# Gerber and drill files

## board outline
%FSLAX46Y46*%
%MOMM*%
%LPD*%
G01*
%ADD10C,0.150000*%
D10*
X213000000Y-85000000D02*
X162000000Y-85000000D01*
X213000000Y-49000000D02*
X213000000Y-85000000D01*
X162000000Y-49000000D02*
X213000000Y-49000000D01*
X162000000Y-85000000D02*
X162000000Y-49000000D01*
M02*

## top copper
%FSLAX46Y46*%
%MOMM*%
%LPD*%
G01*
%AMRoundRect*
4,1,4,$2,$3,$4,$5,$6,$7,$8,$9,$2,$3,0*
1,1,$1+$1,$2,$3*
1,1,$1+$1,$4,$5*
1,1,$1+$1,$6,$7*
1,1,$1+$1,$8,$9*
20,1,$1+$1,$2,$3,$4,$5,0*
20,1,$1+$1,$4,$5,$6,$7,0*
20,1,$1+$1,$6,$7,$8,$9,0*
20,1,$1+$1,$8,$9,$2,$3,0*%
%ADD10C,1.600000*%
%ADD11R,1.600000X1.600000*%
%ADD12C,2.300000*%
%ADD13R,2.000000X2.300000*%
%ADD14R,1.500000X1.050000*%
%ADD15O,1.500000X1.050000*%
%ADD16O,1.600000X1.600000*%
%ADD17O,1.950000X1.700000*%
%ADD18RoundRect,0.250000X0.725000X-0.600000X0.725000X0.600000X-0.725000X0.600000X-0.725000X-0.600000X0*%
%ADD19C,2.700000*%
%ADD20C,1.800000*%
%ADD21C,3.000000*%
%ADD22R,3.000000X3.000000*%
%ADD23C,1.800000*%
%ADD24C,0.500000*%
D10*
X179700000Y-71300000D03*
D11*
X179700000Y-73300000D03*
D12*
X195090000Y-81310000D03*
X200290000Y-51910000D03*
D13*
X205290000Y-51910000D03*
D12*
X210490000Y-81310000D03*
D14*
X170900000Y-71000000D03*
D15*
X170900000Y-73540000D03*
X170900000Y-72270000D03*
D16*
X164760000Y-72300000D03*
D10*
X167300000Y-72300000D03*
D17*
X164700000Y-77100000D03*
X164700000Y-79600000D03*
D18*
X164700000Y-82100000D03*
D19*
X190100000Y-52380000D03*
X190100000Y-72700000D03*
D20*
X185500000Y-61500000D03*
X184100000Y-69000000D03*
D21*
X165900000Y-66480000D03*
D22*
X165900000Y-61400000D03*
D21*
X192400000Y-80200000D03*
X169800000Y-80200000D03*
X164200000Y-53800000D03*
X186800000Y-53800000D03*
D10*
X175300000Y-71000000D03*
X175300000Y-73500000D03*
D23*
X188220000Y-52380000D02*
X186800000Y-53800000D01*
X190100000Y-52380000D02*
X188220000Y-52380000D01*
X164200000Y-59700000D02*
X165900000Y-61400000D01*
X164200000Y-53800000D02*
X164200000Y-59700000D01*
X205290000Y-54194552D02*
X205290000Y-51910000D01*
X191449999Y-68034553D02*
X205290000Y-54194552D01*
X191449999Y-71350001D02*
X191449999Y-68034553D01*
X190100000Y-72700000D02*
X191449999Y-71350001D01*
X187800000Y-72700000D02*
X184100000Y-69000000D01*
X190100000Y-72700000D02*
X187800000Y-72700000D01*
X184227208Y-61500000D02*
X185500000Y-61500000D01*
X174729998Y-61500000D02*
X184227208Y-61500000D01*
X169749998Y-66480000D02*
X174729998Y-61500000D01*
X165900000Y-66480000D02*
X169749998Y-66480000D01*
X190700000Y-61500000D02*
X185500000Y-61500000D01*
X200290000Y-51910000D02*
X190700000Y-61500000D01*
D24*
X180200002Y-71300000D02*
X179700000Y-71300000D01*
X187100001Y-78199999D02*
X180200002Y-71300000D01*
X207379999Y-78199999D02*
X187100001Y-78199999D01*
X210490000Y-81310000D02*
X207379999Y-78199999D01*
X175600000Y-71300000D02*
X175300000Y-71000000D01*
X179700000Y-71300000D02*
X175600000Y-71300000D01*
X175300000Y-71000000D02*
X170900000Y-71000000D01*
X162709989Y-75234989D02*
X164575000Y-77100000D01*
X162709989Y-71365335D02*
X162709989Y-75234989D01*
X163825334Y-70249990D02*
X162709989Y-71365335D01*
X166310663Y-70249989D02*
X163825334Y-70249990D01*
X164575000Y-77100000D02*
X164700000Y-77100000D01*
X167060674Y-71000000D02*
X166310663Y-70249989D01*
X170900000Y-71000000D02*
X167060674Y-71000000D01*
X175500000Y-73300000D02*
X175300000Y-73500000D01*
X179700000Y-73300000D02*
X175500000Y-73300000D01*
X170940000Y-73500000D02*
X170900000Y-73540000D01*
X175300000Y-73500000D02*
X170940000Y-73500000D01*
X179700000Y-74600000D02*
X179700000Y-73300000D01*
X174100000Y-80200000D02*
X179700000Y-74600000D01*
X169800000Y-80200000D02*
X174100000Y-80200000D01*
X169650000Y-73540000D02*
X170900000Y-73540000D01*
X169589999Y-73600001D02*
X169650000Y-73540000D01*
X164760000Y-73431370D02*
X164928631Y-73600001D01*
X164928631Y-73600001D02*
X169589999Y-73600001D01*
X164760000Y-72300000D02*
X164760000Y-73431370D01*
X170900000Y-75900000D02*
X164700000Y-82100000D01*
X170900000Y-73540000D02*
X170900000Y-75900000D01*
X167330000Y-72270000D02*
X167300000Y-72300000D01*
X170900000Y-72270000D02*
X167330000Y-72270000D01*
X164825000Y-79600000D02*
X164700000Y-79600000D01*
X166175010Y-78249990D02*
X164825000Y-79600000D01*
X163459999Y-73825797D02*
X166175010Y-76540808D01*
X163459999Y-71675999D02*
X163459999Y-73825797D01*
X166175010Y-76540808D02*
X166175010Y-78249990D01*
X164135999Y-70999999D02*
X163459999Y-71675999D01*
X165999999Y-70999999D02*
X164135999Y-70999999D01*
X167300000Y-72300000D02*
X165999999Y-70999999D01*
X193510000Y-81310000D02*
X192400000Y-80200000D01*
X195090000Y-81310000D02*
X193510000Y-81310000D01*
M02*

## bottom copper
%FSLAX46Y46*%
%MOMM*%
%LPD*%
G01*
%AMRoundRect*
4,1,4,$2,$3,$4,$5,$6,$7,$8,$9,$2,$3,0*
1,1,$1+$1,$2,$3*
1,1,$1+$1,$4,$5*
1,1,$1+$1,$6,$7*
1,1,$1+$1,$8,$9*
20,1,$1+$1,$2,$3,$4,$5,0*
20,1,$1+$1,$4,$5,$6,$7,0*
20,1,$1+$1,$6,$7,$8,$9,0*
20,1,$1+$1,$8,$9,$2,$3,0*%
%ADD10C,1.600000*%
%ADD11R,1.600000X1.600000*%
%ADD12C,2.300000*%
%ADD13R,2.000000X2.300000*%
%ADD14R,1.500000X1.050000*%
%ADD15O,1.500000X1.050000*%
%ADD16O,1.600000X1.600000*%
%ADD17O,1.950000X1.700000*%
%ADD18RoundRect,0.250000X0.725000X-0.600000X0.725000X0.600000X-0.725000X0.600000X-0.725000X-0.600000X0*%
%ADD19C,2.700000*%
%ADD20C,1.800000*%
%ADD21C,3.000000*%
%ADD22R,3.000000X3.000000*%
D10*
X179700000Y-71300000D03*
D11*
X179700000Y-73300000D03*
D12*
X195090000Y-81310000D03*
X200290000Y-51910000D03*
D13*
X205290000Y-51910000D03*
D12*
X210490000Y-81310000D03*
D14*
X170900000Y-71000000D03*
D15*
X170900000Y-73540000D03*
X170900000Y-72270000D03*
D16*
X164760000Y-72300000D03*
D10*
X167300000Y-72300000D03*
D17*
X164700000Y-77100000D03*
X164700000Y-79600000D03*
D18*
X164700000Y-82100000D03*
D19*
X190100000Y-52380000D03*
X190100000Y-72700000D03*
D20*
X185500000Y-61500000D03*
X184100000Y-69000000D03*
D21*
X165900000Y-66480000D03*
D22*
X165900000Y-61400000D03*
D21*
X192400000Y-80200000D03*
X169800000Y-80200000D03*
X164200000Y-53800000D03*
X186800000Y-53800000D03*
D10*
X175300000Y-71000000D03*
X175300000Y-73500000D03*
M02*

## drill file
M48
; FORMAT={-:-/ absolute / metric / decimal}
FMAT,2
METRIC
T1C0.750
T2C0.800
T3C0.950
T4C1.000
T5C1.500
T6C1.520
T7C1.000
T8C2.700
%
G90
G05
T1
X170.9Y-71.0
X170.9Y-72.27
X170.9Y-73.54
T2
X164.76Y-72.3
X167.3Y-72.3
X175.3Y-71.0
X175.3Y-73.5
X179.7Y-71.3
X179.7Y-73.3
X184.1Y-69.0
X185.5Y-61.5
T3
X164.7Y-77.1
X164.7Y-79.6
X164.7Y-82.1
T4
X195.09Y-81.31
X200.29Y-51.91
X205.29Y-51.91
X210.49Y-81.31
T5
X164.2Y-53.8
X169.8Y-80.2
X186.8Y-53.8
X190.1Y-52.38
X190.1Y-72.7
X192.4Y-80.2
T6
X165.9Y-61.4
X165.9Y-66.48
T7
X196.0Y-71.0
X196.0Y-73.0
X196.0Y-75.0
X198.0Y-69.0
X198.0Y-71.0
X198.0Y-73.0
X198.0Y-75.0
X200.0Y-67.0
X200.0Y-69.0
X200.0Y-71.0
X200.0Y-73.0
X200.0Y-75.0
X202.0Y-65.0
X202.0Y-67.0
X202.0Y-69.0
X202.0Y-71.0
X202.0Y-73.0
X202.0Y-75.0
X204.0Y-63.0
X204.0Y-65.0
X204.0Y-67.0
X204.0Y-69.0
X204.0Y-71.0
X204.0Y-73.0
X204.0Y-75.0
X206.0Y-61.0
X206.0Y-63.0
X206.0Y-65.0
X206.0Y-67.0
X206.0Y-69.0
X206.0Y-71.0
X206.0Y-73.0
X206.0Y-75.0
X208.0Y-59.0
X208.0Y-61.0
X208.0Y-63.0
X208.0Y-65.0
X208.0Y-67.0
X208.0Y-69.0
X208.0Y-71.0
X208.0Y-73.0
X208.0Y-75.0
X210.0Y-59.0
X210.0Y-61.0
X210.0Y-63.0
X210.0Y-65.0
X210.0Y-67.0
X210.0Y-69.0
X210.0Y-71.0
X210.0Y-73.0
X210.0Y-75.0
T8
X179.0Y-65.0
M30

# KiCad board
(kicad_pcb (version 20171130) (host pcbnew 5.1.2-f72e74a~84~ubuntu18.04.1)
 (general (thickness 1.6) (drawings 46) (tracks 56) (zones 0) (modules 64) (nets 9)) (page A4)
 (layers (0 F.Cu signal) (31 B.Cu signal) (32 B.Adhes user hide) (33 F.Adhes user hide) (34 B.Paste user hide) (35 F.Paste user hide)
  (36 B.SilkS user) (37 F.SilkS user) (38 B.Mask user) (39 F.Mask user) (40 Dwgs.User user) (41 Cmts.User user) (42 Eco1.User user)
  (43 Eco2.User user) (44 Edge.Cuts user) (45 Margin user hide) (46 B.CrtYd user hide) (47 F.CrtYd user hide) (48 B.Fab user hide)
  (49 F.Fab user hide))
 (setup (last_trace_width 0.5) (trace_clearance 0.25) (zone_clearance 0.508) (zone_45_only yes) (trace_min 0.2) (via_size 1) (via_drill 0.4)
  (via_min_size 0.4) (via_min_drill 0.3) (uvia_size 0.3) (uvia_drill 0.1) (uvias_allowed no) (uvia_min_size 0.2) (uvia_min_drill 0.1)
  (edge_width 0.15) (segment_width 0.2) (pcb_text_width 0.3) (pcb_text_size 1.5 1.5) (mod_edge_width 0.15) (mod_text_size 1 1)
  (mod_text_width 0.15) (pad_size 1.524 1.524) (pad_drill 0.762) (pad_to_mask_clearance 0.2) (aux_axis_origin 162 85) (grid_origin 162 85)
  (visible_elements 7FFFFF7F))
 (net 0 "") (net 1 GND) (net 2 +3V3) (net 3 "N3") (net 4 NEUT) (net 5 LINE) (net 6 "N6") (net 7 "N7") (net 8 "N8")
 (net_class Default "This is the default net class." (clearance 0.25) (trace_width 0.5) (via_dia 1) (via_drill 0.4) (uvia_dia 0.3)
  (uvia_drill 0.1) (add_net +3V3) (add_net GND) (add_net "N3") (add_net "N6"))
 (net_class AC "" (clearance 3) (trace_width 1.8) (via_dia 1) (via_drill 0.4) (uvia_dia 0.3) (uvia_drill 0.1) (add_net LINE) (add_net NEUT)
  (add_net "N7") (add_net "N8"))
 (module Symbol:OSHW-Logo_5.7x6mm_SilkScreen (layer B.Cu) (at 203.1 79.7 180)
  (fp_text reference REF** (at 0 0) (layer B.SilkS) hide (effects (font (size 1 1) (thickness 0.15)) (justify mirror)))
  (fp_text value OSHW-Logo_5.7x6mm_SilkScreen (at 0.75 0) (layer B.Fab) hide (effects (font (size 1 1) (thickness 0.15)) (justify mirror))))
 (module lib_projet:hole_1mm (layer F.Cu) (at 210 75)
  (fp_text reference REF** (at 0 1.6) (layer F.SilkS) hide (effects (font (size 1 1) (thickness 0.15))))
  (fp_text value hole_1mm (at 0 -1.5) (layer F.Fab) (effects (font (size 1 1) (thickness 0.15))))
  (pad "" np_thru_hole circle (at 0 0) (size 1 1) (drill 1) (layers *.Cu *.Mask)))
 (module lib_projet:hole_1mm (layer F.Cu) (at 208 75)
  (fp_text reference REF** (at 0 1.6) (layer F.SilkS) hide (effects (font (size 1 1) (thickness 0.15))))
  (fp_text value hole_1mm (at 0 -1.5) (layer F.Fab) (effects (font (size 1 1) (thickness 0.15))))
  (pad "" np_thru_hole circle (at 0 0) (size 1 1) (drill 1) (layers *.Cu *.Mask)))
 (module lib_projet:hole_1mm (layer F.Cu) (at 206 75)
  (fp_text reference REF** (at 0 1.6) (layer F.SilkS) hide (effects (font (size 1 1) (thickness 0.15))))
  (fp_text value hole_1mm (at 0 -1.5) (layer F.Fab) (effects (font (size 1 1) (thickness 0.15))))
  (pad "" np_thru_hole circle (at 0 0) (size 1 1) (drill 1) (layers *.Cu *.Mask)))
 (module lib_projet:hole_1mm (layer F.Cu) (at 204 75)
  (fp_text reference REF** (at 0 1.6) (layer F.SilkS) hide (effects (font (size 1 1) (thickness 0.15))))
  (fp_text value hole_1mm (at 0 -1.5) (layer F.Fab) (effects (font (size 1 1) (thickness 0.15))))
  (pad "" np_thru_hole circle (at 0 0) (size 1 1) (drill 1) (layers *.Cu *.Mask)))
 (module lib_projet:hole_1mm (layer F.Cu) (at 202 75)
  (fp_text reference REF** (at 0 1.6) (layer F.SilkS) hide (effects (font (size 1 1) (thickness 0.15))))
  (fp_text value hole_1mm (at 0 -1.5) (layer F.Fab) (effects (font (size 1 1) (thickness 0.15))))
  (pad "" np_thru_hole circle (at 0 0) (size 1 1) (drill 1) (layers *.Cu *.Mask)))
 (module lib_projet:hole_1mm (layer F.Cu) (at 200 75)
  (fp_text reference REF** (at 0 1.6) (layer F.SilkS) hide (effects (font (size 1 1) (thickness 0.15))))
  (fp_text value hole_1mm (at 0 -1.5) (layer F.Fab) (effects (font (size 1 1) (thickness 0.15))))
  (pad "" np_thru_hole circle (at 0 0) (size 1 1) (drill 1) (layers *.Cu *.Mask)))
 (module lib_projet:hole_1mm (layer F.Cu) (at 198 75)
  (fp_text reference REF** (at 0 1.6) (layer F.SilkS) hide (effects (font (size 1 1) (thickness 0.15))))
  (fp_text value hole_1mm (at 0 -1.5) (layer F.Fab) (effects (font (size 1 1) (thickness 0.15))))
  (pad "" np_thru_hole circle (at 0 0) (size 1 1) (drill 1) (layers *.Cu *.Mask)))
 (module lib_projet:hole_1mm (layer F.Cu) (at 196 75)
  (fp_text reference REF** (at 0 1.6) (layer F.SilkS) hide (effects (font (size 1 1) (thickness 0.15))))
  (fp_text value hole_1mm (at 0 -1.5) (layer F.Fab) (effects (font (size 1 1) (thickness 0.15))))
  (pad "" np_thru_hole circle (at 0 0) (size 1 1) (drill 1) (layers *.Cu *.Mask)))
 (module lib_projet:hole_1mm (layer F.Cu) (at 210 73)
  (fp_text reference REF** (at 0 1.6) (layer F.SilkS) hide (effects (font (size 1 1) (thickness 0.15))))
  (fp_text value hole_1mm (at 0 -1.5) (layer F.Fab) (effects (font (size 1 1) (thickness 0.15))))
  (pad "" np_thru_hole circle (at 0 0) (size 1 1) (drill 1) (layers *.Cu *.Mask)))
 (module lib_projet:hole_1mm (layer F.Cu) (at 208 73)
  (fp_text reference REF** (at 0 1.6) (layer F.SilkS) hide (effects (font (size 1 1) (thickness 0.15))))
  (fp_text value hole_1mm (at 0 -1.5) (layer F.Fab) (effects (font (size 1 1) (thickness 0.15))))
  (pad "" np_thru_hole circle (at 0 0) (size 1 1) (drill 1) (layers *.Cu *.Mask)))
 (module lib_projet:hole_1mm (layer F.Cu) (at 206 73)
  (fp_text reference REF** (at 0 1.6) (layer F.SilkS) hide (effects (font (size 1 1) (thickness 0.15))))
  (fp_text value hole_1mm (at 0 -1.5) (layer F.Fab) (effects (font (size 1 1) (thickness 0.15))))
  (pad "" np_thru_hole circle (at 0 0) (size 1 1) (drill 1) (layers *.Cu *.Mask)))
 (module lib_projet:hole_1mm (layer F.Cu) (at 204 73)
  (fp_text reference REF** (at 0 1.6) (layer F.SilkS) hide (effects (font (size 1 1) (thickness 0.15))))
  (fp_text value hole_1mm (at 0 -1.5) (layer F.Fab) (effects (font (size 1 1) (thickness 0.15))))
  (pad "" np_thru_hole circle (at 0 0) (size 1 1) (drill 1) (layers *.Cu *.Mask)))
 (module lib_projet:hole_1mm (layer F.Cu) (at 202 73)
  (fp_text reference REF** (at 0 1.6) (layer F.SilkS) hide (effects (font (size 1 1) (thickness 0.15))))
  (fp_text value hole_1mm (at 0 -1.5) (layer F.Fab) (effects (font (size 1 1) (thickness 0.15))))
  (pad "" np_thru_hole circle (at 0 0) (size 1 1) (drill 1) (layers *.Cu *.Mask)))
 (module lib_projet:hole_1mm (layer F.Cu) (at 200 73)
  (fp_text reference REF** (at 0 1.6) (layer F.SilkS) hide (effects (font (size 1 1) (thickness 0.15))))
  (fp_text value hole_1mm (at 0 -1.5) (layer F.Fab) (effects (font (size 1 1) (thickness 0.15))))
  (pad "" np_thru_hole circle (at 0 0) (size 1 1) (drill 1) (layers *.Cu *.Mask)))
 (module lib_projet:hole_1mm (layer F.Cu) (at 198 73)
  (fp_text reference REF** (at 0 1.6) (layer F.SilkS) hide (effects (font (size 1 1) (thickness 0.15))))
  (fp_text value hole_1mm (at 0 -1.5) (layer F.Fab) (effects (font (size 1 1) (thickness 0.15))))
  (pad "" np_thru_hole circle (at 0 0) (size 1 1) (drill 1) (layers *.Cu *.Mask)))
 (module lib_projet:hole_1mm (layer F.Cu) (at 196 73)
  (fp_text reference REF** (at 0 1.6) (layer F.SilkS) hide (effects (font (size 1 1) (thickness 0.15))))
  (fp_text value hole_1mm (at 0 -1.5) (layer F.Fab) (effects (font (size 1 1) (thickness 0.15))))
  (pad "" np_thru_hole circle (at 0 0) (size 1 1) (drill 1) (layers *.Cu *.Mask)))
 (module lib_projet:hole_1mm (layer F.Cu) (at 210 71)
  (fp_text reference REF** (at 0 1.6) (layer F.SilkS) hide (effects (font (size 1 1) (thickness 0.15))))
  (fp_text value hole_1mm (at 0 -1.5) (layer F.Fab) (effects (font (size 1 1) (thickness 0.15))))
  (pad "" np_thru_hole circle (at 0 0) (size 1 1) (drill 1) (layers *.Cu *.Mask)))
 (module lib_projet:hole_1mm (layer F.Cu) (at 208 71)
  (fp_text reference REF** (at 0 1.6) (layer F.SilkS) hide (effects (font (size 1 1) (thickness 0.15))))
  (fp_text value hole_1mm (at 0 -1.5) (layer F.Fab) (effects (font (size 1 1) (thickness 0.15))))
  (pad "" np_thru_hole circle (at 0 0) (size 1 1) (drill 1) (layers *.Cu *.Mask)))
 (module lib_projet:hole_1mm (layer F.Cu) (at 206 71)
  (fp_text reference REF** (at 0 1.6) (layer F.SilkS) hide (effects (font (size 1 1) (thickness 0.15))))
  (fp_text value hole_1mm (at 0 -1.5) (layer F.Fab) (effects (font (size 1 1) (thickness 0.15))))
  (pad "" np_thru_hole circle (at 0 0) (size 1 1) (drill 1) (layers *.Cu *.Mask)))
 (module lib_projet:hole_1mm (layer F.Cu) (at 204 71)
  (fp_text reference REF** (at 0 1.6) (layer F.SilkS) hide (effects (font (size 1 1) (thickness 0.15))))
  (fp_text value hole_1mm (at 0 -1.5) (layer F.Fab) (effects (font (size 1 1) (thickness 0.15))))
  (pad "" np_thru_hole circle (at 0 0) (size 1 1) (drill 1) (layers *.Cu *.Mask)))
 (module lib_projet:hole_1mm (layer F.Cu) (at 202 71)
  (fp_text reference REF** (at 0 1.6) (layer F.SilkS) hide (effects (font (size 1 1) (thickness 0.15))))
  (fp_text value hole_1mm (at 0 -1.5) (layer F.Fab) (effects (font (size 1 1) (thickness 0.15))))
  (pad "" np_thru_hole circle (at 0 0) (size 1 1) (drill 1) (layers *.Cu *.Mask)))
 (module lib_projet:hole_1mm (layer F.Cu) (at 200 71)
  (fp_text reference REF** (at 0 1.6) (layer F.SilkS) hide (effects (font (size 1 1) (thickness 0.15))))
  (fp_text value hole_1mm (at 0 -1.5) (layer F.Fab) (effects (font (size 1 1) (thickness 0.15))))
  (pad "" np_thru_hole circle (at 0 0) (size 1 1) (drill 1) (layers *.Cu *.Mask)))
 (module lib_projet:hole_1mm (layer F.Cu) (at 198 71)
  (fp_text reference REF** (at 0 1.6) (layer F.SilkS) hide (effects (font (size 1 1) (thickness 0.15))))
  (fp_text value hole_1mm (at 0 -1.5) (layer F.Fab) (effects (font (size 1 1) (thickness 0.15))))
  (pad "" np_thru_hole circle (at 0 0) (size 1 1) (drill 1) (layers *.Cu *.Mask)))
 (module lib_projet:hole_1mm (layer F.Cu) (at 196 71)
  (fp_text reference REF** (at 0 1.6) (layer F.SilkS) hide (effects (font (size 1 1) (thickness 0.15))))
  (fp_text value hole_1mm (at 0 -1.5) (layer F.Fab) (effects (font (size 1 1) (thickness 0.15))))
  (pad "" np_thru_hole circle (at 0 0) (size 1 1) (drill 1) (layers *.Cu *.Mask)))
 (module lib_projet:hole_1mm (layer F.Cu) (at 210 69)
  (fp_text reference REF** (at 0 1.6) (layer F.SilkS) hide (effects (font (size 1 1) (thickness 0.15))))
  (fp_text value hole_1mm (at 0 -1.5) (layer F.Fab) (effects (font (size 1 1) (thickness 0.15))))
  (pad "" np_thru_hole circle (at 0 0) (size 1 1) (drill 1) (layers *.Cu *.Mask)))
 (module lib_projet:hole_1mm (layer F.Cu) (at 208 69)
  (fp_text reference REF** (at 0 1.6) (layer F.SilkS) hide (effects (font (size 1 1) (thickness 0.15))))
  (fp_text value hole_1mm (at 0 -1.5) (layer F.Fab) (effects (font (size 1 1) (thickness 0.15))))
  (pad "" np_thru_hole circle (at 0 0) (size 1 1) (drill 1) (layers *.Cu *.Mask)))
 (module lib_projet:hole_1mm (layer F.Cu) (at 206 69)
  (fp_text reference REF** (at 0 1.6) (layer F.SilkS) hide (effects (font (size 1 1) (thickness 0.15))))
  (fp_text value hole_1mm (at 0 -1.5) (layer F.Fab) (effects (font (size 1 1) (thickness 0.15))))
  (pad "" np_thru_hole circle (at 0 0) (size 1 1) (drill 1) (layers *.Cu *.Mask)))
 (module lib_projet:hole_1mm (layer F.Cu) (at 204 69)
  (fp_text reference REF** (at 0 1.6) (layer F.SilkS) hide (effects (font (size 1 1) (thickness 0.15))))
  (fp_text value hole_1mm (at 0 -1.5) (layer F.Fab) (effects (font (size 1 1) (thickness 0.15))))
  (pad "" np_thru_hole circle (at 0 0) (size 1 1) (drill 1) (layers *.Cu *.Mask)))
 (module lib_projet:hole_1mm (layer F.Cu) (at 202 69)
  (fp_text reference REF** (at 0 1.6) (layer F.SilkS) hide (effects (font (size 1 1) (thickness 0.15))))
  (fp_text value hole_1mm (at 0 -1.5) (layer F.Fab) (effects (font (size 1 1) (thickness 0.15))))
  (pad "" np_thru_hole circle (at 0 0) (size 1 1) (drill 1) (layers *.Cu *.Mask)))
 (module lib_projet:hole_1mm (layer F.Cu) (at 200 69)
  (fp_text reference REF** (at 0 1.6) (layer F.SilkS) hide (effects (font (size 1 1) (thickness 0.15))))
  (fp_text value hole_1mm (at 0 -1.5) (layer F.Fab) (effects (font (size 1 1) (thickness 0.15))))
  (pad "" np_thru_hole circle (at 0 0) (size 1 1) (drill 1) (layers *.Cu *.Mask)))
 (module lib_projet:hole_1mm (layer F.Cu) (at 198 69)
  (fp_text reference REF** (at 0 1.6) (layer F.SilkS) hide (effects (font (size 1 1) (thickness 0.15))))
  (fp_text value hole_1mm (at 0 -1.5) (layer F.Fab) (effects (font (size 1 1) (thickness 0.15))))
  (pad "" np_thru_hole circle (at 0 0) (size 1 1) (drill 1) (layers *.Cu *.Mask)))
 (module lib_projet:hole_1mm (layer F.Cu) (at 210 67)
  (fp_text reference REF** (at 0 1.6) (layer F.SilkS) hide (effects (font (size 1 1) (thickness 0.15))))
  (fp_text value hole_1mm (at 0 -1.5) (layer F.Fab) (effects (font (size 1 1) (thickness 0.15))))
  (pad "" np_thru_hole circle (at 0 0) (size 1 1) (drill 1) (layers *.Cu *.Mask)))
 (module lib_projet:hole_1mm (layer F.Cu) (at 208 67)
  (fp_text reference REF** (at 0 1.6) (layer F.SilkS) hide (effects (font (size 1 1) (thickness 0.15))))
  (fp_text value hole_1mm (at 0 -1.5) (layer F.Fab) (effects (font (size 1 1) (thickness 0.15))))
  (pad "" np_thru_hole circle (at 0 0) (size 1 1) (drill 1) (layers *.Cu *.Mask)))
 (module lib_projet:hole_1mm (layer F.Cu) (at 206 67)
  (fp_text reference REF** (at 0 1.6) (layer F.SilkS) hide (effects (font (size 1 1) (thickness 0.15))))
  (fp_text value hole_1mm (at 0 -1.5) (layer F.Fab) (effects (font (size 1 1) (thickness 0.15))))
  (pad "" np_thru_hole circle (at 0 0) (size 1 1) (drill 1) (layers *.Cu *.Mask)))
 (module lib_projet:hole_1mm (layer F.Cu) (at 204 67)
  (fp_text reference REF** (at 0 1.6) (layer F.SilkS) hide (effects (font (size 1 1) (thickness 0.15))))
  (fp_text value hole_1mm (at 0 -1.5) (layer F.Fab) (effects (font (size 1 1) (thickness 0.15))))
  (pad "" np_thru_hole circle (at 0 0) (size 1 1) (drill 1) (layers *.Cu *.Mask)))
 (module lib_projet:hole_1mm (layer F.Cu) (at 202 67)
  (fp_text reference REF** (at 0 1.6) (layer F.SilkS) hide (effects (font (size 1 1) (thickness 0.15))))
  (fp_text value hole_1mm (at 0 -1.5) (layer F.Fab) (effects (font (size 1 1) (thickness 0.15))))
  (pad "" np_thru_hole circle (at 0 0) (size 1 1) (drill 1) (layers *.Cu *.Mask)))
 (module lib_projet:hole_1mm (layer F.Cu) (at 200 67)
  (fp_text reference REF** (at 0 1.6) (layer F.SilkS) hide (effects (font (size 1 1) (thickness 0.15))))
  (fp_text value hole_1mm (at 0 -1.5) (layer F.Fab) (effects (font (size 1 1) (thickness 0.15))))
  (pad "" np_thru_hole circle (at 0 0) (size 1 1) (drill 1) (layers *.Cu *.Mask)))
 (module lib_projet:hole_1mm (layer F.Cu) (at 210 65)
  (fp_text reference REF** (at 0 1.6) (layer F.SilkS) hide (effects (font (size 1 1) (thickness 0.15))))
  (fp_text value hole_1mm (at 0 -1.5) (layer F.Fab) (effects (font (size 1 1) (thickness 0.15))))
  (pad "" np_thru_hole circle (at 0 0) (size 1 1) (drill 1) (layers *.Cu *.Mask)))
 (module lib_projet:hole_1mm (layer F.Cu) (at 208 65)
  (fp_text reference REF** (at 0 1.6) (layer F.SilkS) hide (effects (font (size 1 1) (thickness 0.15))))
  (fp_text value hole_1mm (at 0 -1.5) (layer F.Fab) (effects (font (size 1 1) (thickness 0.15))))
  (pad "" np_thru_hole circle (at 0 0) (size 1 1) (drill 1) (layers *.Cu *.Mask)))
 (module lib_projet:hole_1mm (layer F.Cu) (at 206 65)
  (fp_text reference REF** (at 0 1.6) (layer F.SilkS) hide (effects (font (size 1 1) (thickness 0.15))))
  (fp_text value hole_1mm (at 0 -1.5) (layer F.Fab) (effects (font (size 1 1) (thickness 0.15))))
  (pad "" np_thru_hole circle (at 0 0) (size 1 1) (drill 1) (layers *.Cu *.Mask)))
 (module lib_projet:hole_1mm (layer F.Cu) (at 204 65)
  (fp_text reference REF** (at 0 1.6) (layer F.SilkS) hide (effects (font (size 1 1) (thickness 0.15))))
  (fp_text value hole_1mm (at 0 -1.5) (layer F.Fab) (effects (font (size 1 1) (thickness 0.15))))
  (pad "" np_thru_hole circle (at 0 0) (size 1 1) (drill 1) (layers *.Cu *.Mask)))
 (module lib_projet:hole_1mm (layer F.Cu) (at 202 65)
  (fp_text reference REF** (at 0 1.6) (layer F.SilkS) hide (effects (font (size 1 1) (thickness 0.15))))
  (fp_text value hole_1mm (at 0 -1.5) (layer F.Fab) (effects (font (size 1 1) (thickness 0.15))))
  (pad "" np_thru_hole circle (at 0 0) (size 1 1) (drill 1) (layers *.Cu *.Mask)))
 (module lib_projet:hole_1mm (layer F.Cu) (at 210 63)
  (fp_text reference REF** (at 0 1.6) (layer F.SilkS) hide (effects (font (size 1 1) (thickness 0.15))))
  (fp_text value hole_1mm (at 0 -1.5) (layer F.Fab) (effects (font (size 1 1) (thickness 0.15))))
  (pad "" np_thru_hole circle (at 0 0) (size 1 1) (drill 1) (layers *.Cu *.Mask)))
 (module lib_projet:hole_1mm (layer F.Cu) (at 208 63)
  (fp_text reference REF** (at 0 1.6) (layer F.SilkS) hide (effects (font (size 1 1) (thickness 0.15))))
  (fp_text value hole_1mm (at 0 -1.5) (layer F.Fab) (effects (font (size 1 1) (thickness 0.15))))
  (pad "" np_thru_hole circle (at 0 0) (size 1 1) (drill 1) (layers *.Cu *.Mask)))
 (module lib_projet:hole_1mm (layer F.Cu) (at 206 63)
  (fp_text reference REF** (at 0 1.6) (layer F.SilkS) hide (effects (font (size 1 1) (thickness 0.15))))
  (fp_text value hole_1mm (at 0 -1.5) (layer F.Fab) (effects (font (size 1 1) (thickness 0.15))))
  (pad "" np_thru_hole circle (at 0 0) (size 1 1) (drill 1) (layers *.Cu *.Mask)))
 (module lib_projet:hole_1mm (layer F.Cu) (at 204 63)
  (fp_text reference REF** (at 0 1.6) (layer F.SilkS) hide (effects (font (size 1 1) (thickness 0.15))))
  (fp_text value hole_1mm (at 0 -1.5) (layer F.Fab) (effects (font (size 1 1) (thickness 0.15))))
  (pad "" np_thru_hole circle (at 0 0) (size 1 1) (drill 1) (layers *.Cu *.Mask)))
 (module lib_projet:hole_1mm (layer F.Cu) (at 210 61)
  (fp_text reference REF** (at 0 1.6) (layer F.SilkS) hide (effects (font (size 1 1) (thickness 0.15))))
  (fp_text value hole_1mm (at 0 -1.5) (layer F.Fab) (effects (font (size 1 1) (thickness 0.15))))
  (pad "" np_thru_hole circle (at 0 0) (size 1 1) (drill 1) (layers *.Cu *.Mask)))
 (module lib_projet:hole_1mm (layer F.Cu) (at 208 61)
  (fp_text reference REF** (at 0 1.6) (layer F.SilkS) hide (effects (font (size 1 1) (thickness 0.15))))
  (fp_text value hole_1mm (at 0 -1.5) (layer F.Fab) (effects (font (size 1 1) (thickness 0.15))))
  (pad "" np_thru_hole circle (at 0 0) (size 1 1) (drill 1) (layers *.Cu *.Mask)))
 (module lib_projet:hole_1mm (layer F.Cu) (at 206 61)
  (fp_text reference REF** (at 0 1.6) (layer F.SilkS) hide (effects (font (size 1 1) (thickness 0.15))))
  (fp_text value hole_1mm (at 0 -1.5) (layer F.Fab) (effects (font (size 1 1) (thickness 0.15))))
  (pad "" np_thru_hole circle (at 0 0) (size 1 1) (drill 1) (layers *.Cu *.Mask)))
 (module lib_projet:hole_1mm (layer F.Cu) (at 210 59)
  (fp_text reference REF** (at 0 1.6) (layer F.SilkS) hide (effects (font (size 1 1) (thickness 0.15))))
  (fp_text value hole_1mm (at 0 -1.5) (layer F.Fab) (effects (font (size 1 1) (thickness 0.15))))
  (pad "" np_thru_hole circle (at 0 0) (size 1 1) (drill 1) (layers *.Cu *.Mask)))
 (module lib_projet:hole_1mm (layer F.Cu) (at 208 59)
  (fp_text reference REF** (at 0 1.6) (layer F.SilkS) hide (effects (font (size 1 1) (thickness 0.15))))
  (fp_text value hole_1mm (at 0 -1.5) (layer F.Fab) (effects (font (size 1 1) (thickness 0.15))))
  (pad "" np_thru_hole circle (at 0 0) (size 1 1) (drill 1) (layers *.Cu *.Mask)))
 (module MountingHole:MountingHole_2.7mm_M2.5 (layer F.Cu) (at 179 65)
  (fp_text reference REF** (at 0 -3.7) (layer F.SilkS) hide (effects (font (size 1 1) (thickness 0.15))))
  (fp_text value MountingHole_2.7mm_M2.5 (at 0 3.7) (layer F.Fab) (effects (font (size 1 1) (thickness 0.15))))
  (pad 1 np_thru_hole circle (at 0 0) (size 2.7 2.7) (drill 2.7) (layers *.Cu *.Mask)))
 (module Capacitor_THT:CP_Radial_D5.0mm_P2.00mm (layer F.Cu) (at 179.7 73.3 90)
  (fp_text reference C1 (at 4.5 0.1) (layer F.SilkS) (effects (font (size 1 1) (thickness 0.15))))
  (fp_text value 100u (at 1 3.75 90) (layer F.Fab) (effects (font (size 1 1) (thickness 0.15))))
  (pad 2 thru_hole circle (at 2 0 90) (size 1.6 1.6) (drill 0.8) (layers *.Cu *.Mask) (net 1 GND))
  (pad 1 thru_hole rect (at 0 0 90) (size 1.6 1.6) (drill 0.8) (layers *.Cu *.Mask) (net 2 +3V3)))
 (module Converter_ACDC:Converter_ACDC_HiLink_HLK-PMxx (layer F.Cu) (at 205.29 51.91 270)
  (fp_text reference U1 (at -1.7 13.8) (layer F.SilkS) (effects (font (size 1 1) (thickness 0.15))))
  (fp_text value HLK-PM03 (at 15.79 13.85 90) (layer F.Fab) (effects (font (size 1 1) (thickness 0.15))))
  (pad 4 thru_hole circle (at 29.4 10.2 270) (size 2.3 2.3) (drill 1) (layers *.Cu *.Mask) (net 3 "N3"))
  (pad 2 thru_hole circle (at 0 5 270) (size 2.3 2.3) (drill 1) (layers *.Cu *.Mask) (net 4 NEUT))
  (pad 1 thru_hole rect (at 0 0 270) (size 2.3 2) (drill 1) (layers *.Cu *.Mask) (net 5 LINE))
  (pad 3 thru_hole circle (at 29.4 -5.2 270) (size 2.3 2.3) (drill 1) (layers *.Cu *.Mask) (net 1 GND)))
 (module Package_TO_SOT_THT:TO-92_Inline (layer F.Cu) (at 170.9 71 270)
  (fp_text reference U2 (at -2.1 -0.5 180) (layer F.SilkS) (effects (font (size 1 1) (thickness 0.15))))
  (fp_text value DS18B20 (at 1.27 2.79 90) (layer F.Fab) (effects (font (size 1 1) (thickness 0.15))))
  (pad 1 thru_hole rect (at 0 0 270) (size 1.05 1.5) (drill 0.75) (layers *.Cu *.Mask) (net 1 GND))
  (pad 3 thru_hole oval (at 2.54 0 270) (size 1.05 1.5) (drill 0.75) (layers *.Cu *.Mask) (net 2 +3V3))
  (pad 2 thru_hole oval (at 1.27 0 270) (size 1.05 1.5) (drill 0.75) (layers *.Cu *.Mask) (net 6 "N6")))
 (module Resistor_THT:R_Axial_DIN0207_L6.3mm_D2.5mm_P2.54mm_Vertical (layer F.Cu) (at 167.3 72.3 180)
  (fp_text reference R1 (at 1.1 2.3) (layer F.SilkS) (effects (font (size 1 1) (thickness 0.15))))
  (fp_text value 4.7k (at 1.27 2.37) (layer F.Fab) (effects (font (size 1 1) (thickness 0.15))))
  (pad 2 thru_hole oval (at 2.54 0 180) (size 1.6 1.6) (drill 0.8) (layers *.Cu *.Mask) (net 2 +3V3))
  (pad 1 thru_hole circle (at 0 0 180) (size 1.6 1.6) (drill 0.8) (layers *.Cu *.Mask) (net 6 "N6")))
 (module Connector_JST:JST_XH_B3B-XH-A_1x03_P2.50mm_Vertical (layer F.Cu) (at 164.7 82.1 90)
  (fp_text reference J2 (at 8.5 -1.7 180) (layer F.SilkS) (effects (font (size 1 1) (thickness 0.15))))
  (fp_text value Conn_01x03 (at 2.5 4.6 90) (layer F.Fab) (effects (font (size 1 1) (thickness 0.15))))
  (pad 3 thru_hole oval (at 5 0 90) (size 1.7 1.95) (drill 0.95) (layers *.Cu *.Mask) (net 1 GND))
  (pad 2 thru_hole oval (at 2.5 0 90) (size 1.7 1.95) (drill 0.95) (layers *.Cu *.Mask) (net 6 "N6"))
  (pad 1 thru_hole roundrect (at 0 0 90) (size 1.7 1.95) (drill 0.95) (layers *.Cu *.Mask) (roundrect_rratio 0.147059) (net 2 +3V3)))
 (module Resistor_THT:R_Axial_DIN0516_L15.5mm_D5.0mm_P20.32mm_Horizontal (layer F.Cu) (at 190.1 72.7 90)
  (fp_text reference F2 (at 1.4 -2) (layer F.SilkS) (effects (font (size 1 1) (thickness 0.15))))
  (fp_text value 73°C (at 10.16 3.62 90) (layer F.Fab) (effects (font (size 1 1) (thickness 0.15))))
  (pad 2 thru_hole circle (at 20.32 0 90) (size 2.7 2.7) (drill 1.5) (layers *.Cu *.Mask) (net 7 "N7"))
  (pad 1 thru_hole circle (at 0 0 90) (size 2.7 2.7) (drill 1.5) (layers *.Cu *.Mask) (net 5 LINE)))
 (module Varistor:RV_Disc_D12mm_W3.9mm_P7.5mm (layer F.Cu) (at 184.1 69 90)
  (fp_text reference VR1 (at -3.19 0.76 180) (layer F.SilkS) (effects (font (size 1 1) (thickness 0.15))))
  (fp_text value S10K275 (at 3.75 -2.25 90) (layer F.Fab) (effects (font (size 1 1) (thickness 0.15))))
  (pad 2 thru_hole circle (at 7.5 1.4 90) (size 1.8 1.8) (drill 0.8) (layers *.Cu *.Mask) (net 4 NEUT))
  (pad 1 thru_hole circle (at 0 0 90) (size 1.8 1.8) (drill 0.8) (layers *.Cu *.Mask) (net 5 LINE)))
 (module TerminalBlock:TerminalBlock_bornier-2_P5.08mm (layer F.Cu) (at 165.9 61.4 270)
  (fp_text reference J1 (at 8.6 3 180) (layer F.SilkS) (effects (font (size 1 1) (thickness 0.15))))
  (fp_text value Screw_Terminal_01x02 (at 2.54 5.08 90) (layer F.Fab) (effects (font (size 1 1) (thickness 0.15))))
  (pad 2 thru_hole circle (at 5.08 0 270) (size 3 3) (drill 1.52) (layers *.Cu *.Mask) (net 4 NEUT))
  (pad 1 thru_hole rect (at 0 0 270) (size 3 3) (drill 1.52) (layers *.Cu *.Mask) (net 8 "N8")))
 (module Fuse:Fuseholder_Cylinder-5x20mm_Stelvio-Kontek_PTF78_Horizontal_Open (layer F.Cu) (at 169.8 80.2)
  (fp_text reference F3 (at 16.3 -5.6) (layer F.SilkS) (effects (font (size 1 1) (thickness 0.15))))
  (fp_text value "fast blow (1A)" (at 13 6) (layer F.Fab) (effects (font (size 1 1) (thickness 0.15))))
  (pad 2 thru_hole circle (at 22.6 0) (size 3 3) (drill 1.5) (layers *.Cu *.Mask) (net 3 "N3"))
  (pad 1 thru_hole circle (at 0 0) (size 3 3) (drill 1.5) (layers *.Cu *.Mask) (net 2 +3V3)))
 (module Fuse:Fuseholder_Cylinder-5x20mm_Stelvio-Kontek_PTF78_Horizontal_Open (layer F.Cu) (at 186.8 53.8 180)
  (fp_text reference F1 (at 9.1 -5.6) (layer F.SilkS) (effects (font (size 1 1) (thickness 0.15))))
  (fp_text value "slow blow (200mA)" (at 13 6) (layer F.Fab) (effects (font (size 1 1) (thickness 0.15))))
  (pad 2 thru_hole circle (at 22.6 0 180) (size 3 3) (drill 1.5) (layers *.Cu *.Mask) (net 8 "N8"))
  (pad 1 thru_hole circle (at 0 0 180) (size 3 3) (drill 1.5) (layers *.Cu *.Mask) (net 7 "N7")))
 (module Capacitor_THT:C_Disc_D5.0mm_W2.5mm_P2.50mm (layer F.Cu) (at 175.3 73.5 90)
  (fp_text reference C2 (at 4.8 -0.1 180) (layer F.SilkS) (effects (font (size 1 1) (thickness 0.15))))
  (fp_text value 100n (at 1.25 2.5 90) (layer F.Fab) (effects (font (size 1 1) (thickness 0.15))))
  (pad 2 thru_hole circle (at 2.5 0 90) (size 1.6 1.6) (drill 0.8) (layers *.Cu *.Mask) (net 1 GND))
  (pad 1 thru_hole circle (at 0 0 90) (size 1.6 1.6) (drill 0.8) (layers *.Cu *.Mask) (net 2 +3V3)))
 (gr_line (start 213 85) (end 162 85) (layer Edge.Cuts) (width 0.15))
 (gr_line (start 213 49) (end 213 85) (layer Edge.Cuts) (width 0.15))
 (gr_line (start 162 49) (end 213 49) (layer Edge.Cuts) (width 0.15))
 (gr_line (start 162 85) (end 162 49) (layer Edge.Cuts) (width 0.15))
 (segment (start 188.22 52.38) (end 186.8 53.8) (width 1.8) (layer F.Cu) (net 7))
 (segment (start 190.1 52.38) (end 188.22 52.38) (width 1.8) (layer F.Cu) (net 7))
 (segment (start 164.2 59.7) (end 165.9 61.4) (width 1.8) (layer F.Cu) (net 8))
 (segment (start 164.2 53.8) (end 164.2 59.7) (width 1.8) (layer F.Cu) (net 8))
 (segment (start 205.29 54.194552) (end 205.29 51.91) (width 1.8) (layer F.Cu) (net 5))
 (segment (start 191.449999 68.034553) (end 205.29 54.194552) (width 1.8) (layer F.Cu) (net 5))
 (segment (start 191.449999 71.350001) (end 191.449999 68.034553) (width 1.8) (layer F.Cu) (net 5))
 (segment (start 190.1 72.7) (end 191.449999 71.350001) (width 1.8) (layer F.Cu) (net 5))
 (segment (start 187.8 72.7) (end 184.1 69) (width 1.8) (layer F.Cu) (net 5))
 (segment (start 190.1 72.7) (end 187.8 72.7) (width 1.8) (layer F.Cu) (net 5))
 (segment (start 184.227208 61.5) (end 185.5 61.5) (width 1.8) (layer F.Cu) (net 4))
 (segment (start 174.729998 61.5) (end 184.227208 61.5) (width 1.8) (layer F.Cu) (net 4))
 (segment (start 169.749998 66.48) (end 174.729998 61.5) (width 1.8) (layer F.Cu) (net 4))
 (segment (start 165.9 66.48) (end 169.749998 66.48) (width 1.8) (layer F.Cu) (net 4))
 (segment (start 190.7 61.5) (end 185.5 61.5) (width 1.8) (layer F.Cu) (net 4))
 (segment (start 200.29 51.91) (end 190.7 61.5) (width 1.8) (layer F.Cu) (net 4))
 (segment (start 180.200002 71.3) (end 179.7 71.3) (width 0.5) (layer F.Cu) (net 1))
 (segment (start 187.100001 78.199999) (end 180.200002 71.3) (width 0.5) (layer F.Cu) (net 1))
 (segment (start 207.379999 78.199999) (end 187.100001 78.199999) (width 0.5) (layer F.Cu) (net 1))
 (segment (start 210.49 81.31) (end 207.379999 78.199999) (width 0.5) (layer F.Cu) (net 1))
 (segment (start 175.6 71.3) (end 175.3 71) (width 0.5) (layer F.Cu) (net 1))
 (segment (start 179.7 71.3) (end 175.6 71.3) (width 0.5) (layer F.Cu) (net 1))
 (segment (start 175.3 71) (end 170.9 71) (width 0.5) (layer F.Cu) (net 1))
 (segment (start 162.709989 75.234989) (end 164.575 77.1) (width 0.5) (layer F.Cu) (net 1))
 (segment (start 162.709989 71.365335) (end 162.709989 75.234989) (width 0.5) (layer F.Cu) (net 1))
 (segment (start 163.825334 70.24999) (end 162.709989 71.365335) (width 0.5) (layer F.Cu) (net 1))
 (segment (start 166.310663 70.249989) (end 163.825334 70.24999) (width 0.5) (layer F.Cu) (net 1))
 (segment (start 164.575 77.1) (end 164.7 77.1) (width 0.5) (layer F.Cu) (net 1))
 (segment (start 167.060674 71) (end 166.310663 70.249989) (width 0.5) (layer F.Cu) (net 1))
 (segment (start 170.9 71) (end 167.060674 71) (width 0.5) (layer F.Cu) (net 1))
 (segment (start 175.5 73.3) (end 175.3 73.5) (width 0.5) (layer F.Cu) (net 2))
 (segment (start 179.7 73.3) (end 175.5 73.3) (width 0.5) (layer F.Cu) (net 2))
 (segment (start 170.94 73.5) (end 170.9 73.54) (width 0.5) (layer F.Cu) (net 2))
 (segment (start 175.3 73.5) (end 170.94 73.5) (width 0.5) (layer F.Cu) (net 2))
 (segment (start 179.7 74.6) (end 179.7 73.3) (width 0.5) (layer F.Cu) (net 2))
 (segment (start 174.1 80.2) (end 179.7 74.6) (width 0.5) (layer F.Cu) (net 2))
 (segment (start 169.8 80.2) (end 174.1 80.2) (width 0.5) (layer F.Cu) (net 2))
 (segment (start 169.65 73.54) (end 170.9 73.54) (width 0.5) (layer F.Cu) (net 2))
 (segment (start 169.589999 73.600001) (end 169.65 73.54) (width 0.5) (layer F.Cu) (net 2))
 (segment (start 164.76 73.43137) (end 164.928631 73.600001) (width 0.5) (layer F.Cu) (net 2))
 (segment (start 164.928631 73.600001) (end 169.589999 73.600001) (width 0.5) (layer F.Cu) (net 2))
 (segment (start 164.76 72.3) (end 164.76 73.43137) (width 0.5) (layer F.Cu) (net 2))
 (segment (start 170.9 75.9) (end 164.7 82.1) (width 0.5) (layer F.Cu) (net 2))
 (segment (start 170.9 73.54) (end 170.9 75.9) (width 0.5) (layer F.Cu) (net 2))
 (segment (start 167.33 72.27) (end 167.3 72.3) (width 0.5) (layer F.Cu) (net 6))
 (segment (start 170.9 72.27) (end 167.33 72.27) (width 0.5) (layer F.Cu) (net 6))
 (segment (start 164.825 79.6) (end 164.7 79.6) (width 0.5) (layer F.Cu) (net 6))
 (segment (start 166.17501 78.24999) (end 164.825 79.6) (width 0.5) (layer F.Cu) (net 6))
 (segment (start 163.459999 73.825797) (end 166.17501 76.540808) (width 0.5) (layer F.Cu) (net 6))
 (segment (start 163.459999 71.675999) (end 163.459999 73.825797) (width 0.5) (layer F.Cu) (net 6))
 (segment (start 166.17501 76.540808) (end 166.17501 78.24999) (width 0.5) (layer F.Cu) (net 6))
 (segment (start 164.135999 70.999999) (end 163.459999 71.675999) (width 0.5) (layer F.Cu) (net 6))
 (segment (start 165.999999 70.999999) (end 164.135999 70.999999) (width 0.5) (layer F.Cu) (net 6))
 (segment (start 167.3 72.3) (end 165.999999 70.999999) (width 0.5) (layer F.Cu) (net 6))
 (segment (start 193.51 81.31) (end 192.4 80.2) (width 0.5) (layer F.Cu) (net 3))
 (segment (start 195.09 81.31) (end 193.51 81.31) (width 0.5) (layer F.Cu) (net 3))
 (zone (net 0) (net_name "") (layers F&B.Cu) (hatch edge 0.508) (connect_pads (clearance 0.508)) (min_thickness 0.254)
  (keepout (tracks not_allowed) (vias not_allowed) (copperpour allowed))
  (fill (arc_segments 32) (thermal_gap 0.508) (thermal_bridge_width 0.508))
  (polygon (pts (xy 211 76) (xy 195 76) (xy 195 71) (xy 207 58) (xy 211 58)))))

